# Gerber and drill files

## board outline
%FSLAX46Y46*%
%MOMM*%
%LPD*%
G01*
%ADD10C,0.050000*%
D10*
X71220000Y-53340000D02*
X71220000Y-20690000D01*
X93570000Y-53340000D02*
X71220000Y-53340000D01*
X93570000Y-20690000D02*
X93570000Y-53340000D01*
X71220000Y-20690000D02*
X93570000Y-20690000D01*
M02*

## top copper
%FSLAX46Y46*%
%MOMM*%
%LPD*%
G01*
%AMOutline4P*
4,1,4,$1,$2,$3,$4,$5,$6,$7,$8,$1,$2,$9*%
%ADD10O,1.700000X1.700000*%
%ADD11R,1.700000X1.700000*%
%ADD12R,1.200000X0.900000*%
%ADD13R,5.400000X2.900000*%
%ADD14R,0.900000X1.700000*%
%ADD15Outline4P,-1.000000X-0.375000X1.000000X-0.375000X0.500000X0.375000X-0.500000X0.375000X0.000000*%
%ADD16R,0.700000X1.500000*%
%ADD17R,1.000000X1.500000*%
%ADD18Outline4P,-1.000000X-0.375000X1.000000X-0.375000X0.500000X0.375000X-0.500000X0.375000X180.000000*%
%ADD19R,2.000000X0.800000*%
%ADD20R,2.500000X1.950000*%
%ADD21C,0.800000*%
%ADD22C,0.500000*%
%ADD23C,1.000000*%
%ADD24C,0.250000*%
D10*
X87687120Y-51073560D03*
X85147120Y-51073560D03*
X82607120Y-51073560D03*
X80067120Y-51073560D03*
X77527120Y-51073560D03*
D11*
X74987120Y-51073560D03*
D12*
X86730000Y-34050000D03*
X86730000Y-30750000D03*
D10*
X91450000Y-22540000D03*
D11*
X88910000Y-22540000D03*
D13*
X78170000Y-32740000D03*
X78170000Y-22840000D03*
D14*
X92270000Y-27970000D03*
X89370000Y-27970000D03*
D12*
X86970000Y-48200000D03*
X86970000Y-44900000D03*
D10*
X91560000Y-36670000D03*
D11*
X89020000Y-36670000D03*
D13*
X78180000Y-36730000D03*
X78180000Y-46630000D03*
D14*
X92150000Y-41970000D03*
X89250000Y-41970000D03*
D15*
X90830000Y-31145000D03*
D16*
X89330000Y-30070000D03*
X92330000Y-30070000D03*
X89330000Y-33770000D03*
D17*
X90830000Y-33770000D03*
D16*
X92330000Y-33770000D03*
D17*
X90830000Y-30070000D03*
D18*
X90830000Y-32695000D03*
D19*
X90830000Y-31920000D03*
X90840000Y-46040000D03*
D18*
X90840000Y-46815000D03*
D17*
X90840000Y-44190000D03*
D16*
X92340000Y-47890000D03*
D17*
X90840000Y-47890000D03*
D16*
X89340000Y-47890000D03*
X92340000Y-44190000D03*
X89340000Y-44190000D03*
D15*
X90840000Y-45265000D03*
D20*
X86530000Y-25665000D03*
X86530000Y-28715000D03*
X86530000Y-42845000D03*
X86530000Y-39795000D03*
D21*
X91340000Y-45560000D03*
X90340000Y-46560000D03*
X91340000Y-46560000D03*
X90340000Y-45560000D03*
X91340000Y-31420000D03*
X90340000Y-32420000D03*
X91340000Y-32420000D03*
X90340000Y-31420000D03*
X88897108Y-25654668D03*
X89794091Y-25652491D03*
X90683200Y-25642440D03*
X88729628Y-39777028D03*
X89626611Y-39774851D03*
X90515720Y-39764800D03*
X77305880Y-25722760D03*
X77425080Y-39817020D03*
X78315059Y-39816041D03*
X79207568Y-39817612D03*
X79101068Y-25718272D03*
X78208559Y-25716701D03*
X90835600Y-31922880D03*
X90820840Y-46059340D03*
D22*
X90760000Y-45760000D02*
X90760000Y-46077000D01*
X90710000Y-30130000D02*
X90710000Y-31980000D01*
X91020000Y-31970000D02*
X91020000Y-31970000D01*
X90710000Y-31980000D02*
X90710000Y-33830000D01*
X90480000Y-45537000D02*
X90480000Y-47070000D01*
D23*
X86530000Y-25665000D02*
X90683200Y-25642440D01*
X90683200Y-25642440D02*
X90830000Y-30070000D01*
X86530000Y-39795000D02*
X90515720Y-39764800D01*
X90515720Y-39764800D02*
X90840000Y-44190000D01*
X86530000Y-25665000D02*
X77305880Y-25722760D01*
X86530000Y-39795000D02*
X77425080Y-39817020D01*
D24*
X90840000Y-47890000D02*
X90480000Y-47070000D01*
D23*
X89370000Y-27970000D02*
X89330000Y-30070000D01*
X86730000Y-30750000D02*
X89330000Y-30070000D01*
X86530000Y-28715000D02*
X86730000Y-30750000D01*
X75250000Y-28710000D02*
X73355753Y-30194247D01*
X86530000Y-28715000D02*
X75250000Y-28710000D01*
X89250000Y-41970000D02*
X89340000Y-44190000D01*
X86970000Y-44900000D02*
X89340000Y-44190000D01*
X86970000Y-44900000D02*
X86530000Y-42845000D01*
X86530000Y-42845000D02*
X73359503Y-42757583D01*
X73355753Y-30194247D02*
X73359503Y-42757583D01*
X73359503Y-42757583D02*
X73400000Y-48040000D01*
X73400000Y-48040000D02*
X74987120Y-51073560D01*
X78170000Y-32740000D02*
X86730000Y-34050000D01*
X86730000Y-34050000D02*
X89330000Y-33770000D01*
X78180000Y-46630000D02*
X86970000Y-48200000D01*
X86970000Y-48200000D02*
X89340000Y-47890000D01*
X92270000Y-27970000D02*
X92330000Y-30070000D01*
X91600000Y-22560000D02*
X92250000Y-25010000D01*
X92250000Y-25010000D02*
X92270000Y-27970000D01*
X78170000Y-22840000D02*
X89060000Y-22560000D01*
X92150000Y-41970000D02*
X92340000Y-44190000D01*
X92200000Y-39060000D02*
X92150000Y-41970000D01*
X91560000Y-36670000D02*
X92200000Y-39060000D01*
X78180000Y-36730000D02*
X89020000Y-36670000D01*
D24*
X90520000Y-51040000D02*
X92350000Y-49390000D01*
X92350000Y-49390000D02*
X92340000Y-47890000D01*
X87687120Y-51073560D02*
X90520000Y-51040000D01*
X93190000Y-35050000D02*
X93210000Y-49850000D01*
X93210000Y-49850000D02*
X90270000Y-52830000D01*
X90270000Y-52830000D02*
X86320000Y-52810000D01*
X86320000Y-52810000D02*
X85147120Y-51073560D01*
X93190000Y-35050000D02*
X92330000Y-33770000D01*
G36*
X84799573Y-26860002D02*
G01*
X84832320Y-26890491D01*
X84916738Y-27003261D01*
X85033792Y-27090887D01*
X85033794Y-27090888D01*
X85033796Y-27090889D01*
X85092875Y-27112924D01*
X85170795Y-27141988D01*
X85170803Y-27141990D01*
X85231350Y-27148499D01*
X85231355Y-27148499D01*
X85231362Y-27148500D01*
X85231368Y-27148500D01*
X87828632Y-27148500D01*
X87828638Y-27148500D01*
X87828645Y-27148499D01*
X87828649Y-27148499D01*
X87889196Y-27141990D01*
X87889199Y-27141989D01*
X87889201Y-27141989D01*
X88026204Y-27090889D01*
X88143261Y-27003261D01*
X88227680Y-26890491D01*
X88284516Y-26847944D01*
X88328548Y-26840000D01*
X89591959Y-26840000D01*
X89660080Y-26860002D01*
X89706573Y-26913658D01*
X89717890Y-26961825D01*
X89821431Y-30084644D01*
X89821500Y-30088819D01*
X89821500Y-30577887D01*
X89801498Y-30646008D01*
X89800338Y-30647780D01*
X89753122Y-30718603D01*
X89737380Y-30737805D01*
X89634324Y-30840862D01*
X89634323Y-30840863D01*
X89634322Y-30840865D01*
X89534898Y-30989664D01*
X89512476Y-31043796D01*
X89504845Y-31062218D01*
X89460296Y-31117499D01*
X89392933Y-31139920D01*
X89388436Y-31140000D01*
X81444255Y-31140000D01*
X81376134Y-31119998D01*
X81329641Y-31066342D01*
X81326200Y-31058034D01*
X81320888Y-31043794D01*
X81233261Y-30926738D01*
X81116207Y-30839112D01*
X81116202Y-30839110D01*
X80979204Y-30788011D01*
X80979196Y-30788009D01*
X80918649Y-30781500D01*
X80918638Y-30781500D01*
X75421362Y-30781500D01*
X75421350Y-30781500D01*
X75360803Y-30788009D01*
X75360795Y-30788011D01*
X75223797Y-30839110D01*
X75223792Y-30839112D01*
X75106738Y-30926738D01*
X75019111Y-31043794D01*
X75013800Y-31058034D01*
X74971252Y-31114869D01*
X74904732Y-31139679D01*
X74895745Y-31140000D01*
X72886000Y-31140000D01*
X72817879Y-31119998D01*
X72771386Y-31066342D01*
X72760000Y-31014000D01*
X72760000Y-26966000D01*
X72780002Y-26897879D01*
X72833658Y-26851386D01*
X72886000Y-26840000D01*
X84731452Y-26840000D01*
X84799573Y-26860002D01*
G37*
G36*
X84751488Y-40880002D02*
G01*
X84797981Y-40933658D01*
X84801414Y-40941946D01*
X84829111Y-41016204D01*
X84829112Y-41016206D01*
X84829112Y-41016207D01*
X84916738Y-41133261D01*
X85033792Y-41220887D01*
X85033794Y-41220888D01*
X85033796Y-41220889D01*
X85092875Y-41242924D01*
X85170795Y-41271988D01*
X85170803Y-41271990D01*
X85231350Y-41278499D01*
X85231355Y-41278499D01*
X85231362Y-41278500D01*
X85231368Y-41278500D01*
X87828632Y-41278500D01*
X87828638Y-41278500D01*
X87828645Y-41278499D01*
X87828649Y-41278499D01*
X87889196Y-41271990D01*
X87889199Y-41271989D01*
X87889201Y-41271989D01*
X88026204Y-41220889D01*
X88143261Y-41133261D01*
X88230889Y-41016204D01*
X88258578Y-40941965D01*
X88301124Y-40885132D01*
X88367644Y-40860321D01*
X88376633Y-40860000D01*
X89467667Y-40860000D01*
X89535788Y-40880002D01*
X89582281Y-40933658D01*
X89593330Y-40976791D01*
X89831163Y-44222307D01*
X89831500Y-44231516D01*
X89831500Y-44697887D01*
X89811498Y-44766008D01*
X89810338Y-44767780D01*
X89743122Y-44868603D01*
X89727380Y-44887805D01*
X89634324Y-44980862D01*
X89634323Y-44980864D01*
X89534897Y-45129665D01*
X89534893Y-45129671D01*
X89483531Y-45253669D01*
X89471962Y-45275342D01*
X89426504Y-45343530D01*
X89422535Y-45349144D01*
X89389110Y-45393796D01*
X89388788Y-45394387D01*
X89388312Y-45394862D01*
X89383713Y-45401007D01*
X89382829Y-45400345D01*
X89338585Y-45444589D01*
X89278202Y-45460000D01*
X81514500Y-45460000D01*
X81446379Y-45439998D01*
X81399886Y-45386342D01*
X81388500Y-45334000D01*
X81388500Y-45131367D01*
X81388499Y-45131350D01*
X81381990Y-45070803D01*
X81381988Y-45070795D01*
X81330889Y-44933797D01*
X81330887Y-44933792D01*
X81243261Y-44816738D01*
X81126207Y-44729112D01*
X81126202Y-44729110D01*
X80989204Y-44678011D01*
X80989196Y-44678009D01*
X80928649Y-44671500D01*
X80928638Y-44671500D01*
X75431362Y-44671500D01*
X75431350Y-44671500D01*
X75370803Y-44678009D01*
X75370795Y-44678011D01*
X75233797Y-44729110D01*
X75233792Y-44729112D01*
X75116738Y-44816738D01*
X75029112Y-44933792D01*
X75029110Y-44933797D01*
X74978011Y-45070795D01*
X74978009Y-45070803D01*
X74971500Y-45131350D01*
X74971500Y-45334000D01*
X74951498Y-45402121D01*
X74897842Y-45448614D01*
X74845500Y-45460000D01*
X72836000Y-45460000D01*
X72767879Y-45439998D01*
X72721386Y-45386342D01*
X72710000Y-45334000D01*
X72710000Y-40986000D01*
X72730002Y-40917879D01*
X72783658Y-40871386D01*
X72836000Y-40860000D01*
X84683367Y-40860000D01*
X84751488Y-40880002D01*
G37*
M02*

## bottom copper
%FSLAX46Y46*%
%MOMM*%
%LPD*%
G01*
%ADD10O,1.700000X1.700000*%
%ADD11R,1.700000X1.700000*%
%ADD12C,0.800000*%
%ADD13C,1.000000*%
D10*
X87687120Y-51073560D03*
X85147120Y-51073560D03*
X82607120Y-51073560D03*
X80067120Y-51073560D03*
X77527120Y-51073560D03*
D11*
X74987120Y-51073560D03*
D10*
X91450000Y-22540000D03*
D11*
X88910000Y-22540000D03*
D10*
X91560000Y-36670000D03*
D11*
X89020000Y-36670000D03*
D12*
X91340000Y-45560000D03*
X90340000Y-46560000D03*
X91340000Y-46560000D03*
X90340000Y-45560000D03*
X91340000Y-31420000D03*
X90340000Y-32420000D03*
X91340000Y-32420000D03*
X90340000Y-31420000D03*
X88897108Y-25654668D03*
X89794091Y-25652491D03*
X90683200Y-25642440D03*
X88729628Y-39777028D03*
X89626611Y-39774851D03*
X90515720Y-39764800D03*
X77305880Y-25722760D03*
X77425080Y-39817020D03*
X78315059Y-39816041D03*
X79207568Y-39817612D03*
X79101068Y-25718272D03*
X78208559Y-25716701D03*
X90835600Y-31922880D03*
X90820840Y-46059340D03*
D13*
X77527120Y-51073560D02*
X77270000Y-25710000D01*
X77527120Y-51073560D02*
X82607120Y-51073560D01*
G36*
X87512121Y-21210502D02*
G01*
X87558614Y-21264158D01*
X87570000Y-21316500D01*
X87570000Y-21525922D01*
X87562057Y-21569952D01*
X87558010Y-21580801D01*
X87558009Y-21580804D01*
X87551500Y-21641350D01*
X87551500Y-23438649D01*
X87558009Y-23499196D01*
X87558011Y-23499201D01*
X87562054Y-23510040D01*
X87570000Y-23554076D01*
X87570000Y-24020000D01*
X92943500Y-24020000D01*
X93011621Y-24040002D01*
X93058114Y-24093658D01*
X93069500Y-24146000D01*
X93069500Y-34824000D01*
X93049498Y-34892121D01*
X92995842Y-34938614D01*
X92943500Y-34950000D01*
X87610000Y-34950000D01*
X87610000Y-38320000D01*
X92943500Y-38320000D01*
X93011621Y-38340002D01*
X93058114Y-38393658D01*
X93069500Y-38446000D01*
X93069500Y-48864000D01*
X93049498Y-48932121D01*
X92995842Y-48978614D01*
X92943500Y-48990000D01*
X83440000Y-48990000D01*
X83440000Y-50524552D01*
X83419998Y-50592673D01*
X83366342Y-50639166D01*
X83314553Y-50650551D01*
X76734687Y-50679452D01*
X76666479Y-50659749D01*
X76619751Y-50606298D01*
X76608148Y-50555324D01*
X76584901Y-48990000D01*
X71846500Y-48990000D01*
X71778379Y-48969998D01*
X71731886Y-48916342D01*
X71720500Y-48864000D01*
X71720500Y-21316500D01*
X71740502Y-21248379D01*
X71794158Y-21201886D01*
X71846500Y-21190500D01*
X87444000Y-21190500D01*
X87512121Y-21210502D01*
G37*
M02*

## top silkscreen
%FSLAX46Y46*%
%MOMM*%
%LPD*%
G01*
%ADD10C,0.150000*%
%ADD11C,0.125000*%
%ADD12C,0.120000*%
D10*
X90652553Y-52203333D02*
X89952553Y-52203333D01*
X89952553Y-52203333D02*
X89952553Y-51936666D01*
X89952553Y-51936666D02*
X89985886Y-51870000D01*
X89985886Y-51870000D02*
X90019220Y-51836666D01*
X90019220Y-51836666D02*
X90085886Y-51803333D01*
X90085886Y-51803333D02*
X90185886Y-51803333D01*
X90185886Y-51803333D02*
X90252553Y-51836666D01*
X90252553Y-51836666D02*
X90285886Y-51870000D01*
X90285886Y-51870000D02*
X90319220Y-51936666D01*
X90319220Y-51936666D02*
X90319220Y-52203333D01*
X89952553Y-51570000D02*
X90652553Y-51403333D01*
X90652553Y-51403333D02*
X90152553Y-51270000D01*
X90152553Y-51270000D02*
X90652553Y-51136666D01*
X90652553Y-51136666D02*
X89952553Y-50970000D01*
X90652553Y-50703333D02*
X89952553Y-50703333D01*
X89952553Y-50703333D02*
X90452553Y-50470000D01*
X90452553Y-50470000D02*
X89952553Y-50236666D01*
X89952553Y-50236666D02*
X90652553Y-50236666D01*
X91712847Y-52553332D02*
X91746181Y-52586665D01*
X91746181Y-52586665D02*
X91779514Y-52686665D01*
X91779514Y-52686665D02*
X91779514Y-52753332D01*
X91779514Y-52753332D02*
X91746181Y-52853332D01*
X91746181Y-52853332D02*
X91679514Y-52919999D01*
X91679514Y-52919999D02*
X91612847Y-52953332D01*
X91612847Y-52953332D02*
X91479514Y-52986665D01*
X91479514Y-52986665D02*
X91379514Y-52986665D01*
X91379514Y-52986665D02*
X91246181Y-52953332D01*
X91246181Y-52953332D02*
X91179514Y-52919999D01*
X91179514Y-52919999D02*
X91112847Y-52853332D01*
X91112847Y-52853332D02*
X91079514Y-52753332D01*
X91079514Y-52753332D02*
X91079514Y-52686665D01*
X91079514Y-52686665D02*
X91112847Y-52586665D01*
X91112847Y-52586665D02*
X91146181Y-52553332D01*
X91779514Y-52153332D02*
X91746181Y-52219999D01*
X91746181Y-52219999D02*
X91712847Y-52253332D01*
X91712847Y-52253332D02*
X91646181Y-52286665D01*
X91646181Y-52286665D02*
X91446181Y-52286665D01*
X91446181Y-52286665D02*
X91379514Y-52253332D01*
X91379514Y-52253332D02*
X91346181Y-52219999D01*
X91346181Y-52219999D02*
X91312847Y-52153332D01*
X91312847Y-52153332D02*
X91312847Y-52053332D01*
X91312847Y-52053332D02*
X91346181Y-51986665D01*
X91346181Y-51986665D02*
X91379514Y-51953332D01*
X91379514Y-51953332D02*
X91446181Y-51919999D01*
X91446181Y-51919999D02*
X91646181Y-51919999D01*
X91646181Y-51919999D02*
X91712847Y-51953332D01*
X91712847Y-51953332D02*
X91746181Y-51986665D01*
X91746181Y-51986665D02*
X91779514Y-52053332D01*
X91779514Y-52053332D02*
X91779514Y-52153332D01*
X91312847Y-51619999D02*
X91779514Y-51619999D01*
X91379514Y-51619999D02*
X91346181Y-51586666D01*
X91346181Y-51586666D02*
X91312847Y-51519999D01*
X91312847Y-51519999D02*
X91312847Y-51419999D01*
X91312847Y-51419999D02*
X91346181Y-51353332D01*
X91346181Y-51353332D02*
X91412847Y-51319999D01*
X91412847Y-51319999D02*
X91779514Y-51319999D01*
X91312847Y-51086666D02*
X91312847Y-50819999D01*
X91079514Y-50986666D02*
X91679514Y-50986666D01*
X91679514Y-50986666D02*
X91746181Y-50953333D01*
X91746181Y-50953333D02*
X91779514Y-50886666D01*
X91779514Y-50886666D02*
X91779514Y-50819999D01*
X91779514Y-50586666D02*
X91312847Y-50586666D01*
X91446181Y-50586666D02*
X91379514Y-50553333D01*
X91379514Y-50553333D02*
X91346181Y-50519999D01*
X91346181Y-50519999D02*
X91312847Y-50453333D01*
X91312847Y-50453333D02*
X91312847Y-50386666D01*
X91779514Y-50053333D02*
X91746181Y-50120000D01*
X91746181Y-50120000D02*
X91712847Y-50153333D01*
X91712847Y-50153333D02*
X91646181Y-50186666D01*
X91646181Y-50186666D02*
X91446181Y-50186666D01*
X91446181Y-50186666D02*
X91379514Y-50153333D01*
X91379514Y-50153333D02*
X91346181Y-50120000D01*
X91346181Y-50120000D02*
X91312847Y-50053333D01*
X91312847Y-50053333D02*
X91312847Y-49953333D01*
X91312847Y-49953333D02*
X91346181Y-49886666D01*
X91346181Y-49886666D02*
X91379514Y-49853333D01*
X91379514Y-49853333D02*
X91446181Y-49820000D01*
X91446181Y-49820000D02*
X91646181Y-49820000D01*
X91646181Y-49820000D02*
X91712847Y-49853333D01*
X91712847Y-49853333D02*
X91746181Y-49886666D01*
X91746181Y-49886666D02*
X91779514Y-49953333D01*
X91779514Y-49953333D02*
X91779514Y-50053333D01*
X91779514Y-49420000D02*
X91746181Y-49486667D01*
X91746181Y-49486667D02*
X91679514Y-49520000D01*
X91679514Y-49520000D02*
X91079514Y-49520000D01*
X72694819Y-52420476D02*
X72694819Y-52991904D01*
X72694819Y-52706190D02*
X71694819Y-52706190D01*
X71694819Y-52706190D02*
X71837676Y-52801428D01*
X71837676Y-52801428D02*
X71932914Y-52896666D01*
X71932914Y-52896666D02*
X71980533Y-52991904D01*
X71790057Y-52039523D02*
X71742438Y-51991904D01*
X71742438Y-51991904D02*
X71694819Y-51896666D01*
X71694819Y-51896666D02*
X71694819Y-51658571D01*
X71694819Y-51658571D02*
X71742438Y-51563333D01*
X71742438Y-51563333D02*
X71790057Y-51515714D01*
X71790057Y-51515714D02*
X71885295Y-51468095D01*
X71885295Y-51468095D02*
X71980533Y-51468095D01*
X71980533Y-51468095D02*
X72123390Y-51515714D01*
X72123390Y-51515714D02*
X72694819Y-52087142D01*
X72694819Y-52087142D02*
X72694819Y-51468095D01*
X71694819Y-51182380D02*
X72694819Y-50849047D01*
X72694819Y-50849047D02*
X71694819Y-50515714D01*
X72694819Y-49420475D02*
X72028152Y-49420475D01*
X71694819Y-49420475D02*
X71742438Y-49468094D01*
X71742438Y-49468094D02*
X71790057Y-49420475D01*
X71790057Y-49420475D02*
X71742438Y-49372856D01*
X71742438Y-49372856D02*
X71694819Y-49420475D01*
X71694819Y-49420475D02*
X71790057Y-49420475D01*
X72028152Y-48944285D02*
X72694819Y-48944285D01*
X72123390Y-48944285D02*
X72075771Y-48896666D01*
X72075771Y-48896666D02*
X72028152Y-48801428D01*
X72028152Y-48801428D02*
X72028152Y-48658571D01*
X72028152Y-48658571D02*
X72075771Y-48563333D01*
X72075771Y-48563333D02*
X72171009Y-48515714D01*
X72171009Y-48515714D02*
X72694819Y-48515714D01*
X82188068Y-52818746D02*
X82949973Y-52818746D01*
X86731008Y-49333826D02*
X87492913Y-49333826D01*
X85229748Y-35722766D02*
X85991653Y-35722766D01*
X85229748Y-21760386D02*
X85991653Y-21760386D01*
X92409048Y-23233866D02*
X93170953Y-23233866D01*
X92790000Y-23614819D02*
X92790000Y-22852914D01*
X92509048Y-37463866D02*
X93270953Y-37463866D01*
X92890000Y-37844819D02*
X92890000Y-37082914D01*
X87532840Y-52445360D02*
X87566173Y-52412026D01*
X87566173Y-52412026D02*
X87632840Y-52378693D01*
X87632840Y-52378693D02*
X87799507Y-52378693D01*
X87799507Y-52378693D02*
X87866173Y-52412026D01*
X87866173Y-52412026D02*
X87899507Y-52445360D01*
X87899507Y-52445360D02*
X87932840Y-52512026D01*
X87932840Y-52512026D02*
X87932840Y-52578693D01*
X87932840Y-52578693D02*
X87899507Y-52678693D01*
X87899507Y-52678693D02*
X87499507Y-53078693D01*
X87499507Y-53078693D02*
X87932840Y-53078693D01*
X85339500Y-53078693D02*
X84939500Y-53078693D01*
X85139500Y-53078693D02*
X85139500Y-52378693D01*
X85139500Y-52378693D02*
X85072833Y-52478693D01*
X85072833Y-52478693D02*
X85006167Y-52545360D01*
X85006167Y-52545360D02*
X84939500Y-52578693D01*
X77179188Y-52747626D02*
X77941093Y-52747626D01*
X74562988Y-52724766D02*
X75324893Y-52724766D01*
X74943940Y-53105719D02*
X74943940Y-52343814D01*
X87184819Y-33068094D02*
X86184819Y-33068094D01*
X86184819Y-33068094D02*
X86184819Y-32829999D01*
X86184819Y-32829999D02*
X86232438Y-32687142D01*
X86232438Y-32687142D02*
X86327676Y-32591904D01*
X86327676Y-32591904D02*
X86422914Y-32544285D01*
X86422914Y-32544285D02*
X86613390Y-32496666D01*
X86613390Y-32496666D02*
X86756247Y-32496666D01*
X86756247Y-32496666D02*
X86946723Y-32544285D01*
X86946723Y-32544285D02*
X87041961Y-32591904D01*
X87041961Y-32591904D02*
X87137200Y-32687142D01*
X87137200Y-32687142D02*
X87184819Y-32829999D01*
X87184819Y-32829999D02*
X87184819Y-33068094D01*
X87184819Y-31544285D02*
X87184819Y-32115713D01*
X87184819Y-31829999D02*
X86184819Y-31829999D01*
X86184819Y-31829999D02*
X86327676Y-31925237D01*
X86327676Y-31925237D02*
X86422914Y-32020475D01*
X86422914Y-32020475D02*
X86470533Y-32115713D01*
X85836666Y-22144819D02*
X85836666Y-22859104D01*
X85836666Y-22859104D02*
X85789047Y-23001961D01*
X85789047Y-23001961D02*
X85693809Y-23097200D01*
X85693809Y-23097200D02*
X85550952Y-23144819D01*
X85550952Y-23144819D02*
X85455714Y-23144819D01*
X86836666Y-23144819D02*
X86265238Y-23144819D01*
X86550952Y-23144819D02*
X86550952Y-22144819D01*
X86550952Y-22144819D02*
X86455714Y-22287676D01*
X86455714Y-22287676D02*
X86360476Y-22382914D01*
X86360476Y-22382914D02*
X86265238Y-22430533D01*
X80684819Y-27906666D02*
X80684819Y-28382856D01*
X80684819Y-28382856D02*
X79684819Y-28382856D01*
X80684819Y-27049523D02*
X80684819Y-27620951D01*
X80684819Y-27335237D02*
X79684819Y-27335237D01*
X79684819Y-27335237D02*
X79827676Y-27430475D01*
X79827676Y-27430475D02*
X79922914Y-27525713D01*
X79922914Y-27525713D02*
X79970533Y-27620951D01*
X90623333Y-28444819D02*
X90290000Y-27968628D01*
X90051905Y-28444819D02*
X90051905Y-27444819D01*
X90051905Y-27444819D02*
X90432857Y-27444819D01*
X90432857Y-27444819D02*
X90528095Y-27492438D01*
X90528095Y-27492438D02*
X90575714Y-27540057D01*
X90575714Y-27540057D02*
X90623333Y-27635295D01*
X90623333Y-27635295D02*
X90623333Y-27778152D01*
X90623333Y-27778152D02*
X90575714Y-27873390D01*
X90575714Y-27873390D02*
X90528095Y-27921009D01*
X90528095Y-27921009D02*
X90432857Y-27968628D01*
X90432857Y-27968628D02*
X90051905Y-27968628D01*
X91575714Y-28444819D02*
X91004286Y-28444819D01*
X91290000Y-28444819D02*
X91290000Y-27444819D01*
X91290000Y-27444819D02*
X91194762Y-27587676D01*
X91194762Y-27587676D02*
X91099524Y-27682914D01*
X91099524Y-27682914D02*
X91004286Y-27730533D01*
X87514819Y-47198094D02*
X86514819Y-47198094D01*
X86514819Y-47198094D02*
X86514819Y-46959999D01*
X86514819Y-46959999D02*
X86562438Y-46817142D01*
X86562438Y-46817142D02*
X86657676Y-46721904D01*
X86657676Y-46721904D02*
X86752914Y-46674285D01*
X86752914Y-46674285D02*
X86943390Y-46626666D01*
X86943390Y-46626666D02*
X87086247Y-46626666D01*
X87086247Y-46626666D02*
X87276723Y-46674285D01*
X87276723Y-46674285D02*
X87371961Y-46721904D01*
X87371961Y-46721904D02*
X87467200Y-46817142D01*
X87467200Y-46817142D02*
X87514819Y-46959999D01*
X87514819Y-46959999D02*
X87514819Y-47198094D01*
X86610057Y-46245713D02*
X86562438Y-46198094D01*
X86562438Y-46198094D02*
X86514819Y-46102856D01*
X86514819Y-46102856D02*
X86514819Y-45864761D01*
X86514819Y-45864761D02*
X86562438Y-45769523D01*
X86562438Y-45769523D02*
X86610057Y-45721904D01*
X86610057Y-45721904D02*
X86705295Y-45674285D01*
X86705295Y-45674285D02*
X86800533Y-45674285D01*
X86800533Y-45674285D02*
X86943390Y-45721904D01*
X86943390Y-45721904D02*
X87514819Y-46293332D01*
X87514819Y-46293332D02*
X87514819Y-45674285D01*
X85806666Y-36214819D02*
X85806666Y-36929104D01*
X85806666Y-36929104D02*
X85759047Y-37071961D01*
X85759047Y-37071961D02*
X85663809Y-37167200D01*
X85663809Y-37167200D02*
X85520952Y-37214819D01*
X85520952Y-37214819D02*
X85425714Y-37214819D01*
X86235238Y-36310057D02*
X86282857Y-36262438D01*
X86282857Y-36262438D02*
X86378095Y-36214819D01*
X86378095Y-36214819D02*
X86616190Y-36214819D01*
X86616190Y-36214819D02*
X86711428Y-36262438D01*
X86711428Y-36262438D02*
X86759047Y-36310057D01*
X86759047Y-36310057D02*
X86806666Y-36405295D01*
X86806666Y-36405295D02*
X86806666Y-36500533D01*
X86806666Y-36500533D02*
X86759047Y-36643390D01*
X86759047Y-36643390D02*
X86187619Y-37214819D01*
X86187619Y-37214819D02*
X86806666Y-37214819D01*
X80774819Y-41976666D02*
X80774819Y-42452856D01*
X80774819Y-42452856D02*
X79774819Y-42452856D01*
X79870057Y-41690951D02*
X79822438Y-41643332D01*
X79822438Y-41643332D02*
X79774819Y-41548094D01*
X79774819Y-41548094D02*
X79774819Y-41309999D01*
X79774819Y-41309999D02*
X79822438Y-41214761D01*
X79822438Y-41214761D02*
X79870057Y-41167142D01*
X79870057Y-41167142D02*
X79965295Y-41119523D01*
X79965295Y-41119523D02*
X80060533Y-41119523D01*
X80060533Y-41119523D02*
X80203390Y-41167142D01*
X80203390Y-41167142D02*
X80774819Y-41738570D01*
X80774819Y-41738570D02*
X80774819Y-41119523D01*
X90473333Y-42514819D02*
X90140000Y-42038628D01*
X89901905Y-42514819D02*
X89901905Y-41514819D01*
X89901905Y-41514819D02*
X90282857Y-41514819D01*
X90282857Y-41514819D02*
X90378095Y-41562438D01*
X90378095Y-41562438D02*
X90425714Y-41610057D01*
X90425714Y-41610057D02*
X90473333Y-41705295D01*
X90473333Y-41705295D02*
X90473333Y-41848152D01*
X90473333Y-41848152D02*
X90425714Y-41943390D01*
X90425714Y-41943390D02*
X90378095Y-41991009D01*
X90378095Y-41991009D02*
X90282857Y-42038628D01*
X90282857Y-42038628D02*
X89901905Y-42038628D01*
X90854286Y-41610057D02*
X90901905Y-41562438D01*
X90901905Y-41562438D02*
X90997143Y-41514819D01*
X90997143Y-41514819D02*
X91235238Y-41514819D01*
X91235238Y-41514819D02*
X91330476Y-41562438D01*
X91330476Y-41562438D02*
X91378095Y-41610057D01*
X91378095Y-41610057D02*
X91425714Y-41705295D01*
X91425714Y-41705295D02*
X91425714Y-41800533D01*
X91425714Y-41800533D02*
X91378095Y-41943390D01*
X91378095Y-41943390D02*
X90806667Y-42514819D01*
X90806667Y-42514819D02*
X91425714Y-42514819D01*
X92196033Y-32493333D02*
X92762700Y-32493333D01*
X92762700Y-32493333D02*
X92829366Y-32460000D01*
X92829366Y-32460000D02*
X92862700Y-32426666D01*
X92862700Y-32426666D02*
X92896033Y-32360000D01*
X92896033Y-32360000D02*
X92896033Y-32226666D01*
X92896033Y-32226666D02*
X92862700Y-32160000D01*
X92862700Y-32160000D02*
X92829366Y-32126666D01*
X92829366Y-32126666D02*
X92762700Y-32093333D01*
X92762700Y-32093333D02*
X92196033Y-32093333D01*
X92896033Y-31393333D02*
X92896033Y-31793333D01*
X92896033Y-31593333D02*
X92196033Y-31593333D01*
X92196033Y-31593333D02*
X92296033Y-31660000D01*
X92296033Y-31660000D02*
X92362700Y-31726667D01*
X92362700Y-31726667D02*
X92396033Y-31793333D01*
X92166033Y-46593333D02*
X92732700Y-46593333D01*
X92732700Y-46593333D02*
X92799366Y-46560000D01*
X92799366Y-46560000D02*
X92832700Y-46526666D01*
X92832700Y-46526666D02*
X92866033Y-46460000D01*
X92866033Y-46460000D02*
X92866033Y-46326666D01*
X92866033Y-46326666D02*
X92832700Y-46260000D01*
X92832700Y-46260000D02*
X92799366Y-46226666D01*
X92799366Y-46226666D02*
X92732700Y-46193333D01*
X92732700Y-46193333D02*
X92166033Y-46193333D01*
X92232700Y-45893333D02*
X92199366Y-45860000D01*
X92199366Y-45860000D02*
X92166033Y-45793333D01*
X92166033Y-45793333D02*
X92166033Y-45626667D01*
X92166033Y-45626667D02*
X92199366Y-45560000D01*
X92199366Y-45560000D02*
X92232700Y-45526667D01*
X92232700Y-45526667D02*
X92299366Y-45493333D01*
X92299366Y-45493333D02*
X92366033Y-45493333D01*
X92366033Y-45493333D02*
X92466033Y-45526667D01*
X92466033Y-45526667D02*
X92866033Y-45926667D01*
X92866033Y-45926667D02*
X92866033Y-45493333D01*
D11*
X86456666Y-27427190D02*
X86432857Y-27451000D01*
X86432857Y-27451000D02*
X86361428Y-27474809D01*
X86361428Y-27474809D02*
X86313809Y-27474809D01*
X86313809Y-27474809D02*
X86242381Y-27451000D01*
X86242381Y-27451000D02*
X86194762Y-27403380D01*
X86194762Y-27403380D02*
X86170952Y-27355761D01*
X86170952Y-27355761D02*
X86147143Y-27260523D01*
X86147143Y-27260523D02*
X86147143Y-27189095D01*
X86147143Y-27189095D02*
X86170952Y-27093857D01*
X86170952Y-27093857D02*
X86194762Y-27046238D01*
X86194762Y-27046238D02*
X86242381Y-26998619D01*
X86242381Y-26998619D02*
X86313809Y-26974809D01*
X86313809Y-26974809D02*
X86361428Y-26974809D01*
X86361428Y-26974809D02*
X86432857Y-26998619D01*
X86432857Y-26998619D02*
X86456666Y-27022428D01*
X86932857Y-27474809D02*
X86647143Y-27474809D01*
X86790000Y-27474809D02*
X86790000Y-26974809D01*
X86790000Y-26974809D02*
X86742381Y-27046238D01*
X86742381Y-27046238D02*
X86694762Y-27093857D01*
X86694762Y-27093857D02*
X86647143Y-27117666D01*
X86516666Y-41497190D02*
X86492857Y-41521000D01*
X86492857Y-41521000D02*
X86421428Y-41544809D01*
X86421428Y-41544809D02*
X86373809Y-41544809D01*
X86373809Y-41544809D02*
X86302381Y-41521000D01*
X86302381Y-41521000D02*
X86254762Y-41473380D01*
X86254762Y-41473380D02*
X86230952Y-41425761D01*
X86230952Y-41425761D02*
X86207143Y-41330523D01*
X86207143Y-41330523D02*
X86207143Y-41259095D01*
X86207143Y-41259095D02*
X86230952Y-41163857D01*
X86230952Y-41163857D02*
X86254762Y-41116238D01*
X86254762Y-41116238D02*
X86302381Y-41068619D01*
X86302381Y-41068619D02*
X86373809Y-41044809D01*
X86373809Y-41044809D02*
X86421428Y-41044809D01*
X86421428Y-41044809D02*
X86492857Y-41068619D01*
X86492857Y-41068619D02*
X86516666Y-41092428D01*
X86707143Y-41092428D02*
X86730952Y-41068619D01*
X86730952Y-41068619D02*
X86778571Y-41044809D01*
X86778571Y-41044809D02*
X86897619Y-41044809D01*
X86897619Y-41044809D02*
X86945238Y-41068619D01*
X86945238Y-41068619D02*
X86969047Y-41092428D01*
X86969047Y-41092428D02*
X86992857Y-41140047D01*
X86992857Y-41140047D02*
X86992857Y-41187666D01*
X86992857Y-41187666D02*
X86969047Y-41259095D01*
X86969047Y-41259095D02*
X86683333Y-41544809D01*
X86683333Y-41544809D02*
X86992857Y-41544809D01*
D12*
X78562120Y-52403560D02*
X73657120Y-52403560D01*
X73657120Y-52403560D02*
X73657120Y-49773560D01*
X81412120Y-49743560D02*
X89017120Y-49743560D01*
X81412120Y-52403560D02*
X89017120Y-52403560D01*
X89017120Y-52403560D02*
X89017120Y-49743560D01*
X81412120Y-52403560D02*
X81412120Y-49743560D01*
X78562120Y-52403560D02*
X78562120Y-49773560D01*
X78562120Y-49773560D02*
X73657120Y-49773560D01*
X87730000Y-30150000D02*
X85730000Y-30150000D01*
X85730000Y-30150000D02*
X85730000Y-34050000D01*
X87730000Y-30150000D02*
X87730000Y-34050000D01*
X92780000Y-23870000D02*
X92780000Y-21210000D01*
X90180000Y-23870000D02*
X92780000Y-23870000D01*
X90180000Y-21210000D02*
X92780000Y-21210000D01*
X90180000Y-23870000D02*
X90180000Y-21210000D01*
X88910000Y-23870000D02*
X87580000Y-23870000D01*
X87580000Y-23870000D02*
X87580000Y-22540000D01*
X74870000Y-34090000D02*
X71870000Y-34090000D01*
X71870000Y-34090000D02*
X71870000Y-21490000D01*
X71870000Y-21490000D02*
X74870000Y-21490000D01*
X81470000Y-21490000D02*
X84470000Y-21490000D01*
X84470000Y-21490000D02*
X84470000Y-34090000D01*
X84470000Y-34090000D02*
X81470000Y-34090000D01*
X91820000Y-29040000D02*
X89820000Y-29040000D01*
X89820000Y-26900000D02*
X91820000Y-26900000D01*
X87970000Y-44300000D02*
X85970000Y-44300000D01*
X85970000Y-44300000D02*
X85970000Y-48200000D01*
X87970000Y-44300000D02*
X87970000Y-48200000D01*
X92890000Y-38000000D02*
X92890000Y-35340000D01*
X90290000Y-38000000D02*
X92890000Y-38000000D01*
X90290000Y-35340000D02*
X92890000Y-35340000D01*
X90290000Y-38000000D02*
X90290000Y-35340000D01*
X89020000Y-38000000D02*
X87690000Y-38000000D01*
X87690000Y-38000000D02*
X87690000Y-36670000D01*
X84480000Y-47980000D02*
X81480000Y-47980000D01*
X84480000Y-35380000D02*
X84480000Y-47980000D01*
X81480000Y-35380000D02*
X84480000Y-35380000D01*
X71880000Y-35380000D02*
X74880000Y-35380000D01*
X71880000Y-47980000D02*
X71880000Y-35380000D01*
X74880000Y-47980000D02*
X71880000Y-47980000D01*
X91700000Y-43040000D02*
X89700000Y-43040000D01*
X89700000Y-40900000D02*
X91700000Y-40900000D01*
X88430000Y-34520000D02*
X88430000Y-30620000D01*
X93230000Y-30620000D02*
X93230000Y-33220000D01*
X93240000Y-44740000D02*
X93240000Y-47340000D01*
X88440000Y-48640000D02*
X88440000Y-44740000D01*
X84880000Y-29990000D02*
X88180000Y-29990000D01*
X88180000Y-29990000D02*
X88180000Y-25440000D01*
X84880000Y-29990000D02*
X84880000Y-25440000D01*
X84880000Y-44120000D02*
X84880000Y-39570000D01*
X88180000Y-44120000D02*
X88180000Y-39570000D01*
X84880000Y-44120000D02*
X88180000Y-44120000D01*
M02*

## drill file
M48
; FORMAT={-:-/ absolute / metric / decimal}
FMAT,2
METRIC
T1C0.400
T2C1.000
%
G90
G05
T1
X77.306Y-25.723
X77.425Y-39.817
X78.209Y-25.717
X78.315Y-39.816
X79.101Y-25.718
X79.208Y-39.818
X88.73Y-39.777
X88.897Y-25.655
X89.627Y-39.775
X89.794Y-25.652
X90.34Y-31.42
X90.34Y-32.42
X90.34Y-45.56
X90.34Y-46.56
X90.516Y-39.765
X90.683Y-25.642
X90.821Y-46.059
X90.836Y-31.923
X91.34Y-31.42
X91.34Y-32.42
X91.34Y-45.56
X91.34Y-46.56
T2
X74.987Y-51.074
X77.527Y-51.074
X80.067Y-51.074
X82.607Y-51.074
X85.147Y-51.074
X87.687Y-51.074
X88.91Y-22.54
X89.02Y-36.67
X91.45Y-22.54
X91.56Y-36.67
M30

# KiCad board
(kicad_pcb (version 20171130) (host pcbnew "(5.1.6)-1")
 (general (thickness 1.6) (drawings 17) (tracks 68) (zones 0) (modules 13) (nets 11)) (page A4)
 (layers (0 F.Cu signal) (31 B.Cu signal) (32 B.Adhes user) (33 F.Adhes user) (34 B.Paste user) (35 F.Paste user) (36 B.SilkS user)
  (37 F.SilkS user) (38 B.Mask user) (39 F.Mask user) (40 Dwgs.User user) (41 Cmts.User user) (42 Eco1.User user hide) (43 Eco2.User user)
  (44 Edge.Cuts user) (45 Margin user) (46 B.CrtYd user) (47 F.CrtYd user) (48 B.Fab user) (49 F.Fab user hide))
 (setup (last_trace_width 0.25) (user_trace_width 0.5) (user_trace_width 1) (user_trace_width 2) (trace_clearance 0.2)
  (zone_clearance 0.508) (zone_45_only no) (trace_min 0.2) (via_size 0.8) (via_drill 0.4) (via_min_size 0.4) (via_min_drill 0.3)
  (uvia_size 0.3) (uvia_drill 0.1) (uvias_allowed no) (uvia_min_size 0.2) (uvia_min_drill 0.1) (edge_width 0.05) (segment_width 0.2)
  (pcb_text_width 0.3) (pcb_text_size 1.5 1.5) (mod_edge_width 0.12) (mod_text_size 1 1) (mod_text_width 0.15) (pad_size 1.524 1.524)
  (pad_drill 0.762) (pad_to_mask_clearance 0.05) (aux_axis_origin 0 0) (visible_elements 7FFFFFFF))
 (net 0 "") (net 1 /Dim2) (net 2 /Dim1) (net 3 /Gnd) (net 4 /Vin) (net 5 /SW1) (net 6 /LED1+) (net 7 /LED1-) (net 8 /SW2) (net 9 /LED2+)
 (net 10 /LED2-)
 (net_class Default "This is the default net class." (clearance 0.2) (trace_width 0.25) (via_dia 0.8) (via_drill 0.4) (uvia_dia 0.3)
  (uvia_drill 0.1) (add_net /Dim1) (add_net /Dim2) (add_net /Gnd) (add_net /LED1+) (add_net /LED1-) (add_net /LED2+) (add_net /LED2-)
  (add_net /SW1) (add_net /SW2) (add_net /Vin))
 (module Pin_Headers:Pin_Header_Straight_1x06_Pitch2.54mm (layer F.Cu) (at 74.98712 51.07356 90)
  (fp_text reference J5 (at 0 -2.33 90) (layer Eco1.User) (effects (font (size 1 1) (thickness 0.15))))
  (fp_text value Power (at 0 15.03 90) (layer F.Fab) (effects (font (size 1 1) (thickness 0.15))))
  (fp_line (start -1.33 3.575) (end -1.33 -1.33) (layer F.SilkS) (width 0.12))
  (fp_line (start -1.33 -1.33) (end 1.3 -1.33) (layer F.SilkS) (width 0.12))
  (fp_line (start 1.33 6.425) (end 1.33 14.03) (layer F.SilkS) (width 0.12))
  (fp_line (start -1.33 6.425) (end -1.33 14.03) (layer F.SilkS) (width 0.12))
  (fp_line (start -1.33 14.03) (end 1.33 14.03) (layer F.SilkS) (width 0.12))
  (fp_line (start -1.33 6.425) (end 1.33 6.425) (layer F.SilkS) (width 0.12))
  (fp_line (start -1.33 3.575) (end 1.3 3.575) (layer F.SilkS) (width 0.12))
  (fp_line (start 1.3 3.575) (end 1.3 -1.33) (layer F.SilkS) (width 0.12))
  (pad 6 thru_hole oval (at 0 12.7 90) (size 1.7 1.7) (drill 1) (layers *.Cu *.Mask) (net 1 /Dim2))
  (pad 5 thru_hole oval (at 0 10.16 90) (size 1.7 1.7) (drill 1) (layers *.Cu *.Mask) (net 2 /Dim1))
  (pad 4 thru_hole oval (at 0 7.62 90) (size 1.7 1.7) (drill 1) (layers *.Cu *.Mask) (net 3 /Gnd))
  (pad 3 thru_hole oval (at 0 5.08 90) (size 1.7 1.7) (drill 1) (layers *.Cu *.Mask) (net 3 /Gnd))
  (pad 2 thru_hole oval (at 0 2.54 90) (size 1.7 1.7) (drill 1) (layers *.Cu *.Mask) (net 3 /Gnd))
  (pad 1 thru_hole rect (at 0 0 90) (size 1.7 1.7) (drill 1) (layers *.Cu *.Mask) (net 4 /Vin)))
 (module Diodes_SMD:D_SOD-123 (layer F.Cu) (at 86.73 32.4 270)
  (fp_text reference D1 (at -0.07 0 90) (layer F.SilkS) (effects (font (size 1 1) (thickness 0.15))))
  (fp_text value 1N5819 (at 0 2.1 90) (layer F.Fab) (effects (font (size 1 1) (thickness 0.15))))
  (fp_line (start -2.25 -1) (end -2.25 1) (layer F.SilkS) (width 0.12))
  (fp_line (start -2.25 1) (end 1.65 1) (layer F.SilkS) (width 0.12))
  (fp_line (start -2.25 -1) (end 1.65 -1) (layer F.SilkS) (width 0.12))
  (pad 2 smd rect (at 1.65 0 270) (size 0.9 1.2) (layers F.Cu F.Paste F.Mask) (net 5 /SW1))
  (pad 1 smd rect (at -1.65 0 270) (size 0.9 1.2) (layers F.Cu F.Paste F.Mask) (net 4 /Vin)))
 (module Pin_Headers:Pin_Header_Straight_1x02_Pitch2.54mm (layer F.Cu) (at 88.91 22.54 90)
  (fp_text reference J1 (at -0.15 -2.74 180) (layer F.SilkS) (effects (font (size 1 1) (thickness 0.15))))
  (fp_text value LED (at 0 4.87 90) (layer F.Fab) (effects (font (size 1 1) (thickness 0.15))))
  (fp_line (start -1.33 3.87) (end 1.33 3.87) (layer F.SilkS) (width 0.12))
  (fp_line (start -1.33 1.27) (end -1.33 3.87) (layer F.SilkS) (width 0.12))
  (fp_line (start 1.33 1.27) (end 1.33 3.87) (layer F.SilkS) (width 0.12))
  (fp_line (start -1.33 1.27) (end 1.33 1.27) (layer F.SilkS) (width 0.12))
  (fp_line (start -1.33 0) (end -1.33 -1.33) (layer F.SilkS) (width 0.12))
  (fp_line (start -1.33 -1.33) (end 0 -1.33) (layer F.SilkS) (width 0.12))
  (pad 2 thru_hole oval (at 0 2.54 90) (size 1.7 1.7) (drill 1) (layers *.Cu *.Mask) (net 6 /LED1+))
  (pad 1 thru_hole rect (at 0 0 90) (size 1.7 1.7) (drill 1) (layers *.Cu *.Mask) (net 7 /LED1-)))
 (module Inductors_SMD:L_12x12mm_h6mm (layer F.Cu) (at 78.17 27.79 270)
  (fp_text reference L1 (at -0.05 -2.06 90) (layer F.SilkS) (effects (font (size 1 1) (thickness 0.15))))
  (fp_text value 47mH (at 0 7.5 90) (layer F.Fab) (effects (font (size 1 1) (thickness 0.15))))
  (fp_line (start 6.3 3.3) (end 6.3 6.3) (layer F.SilkS) (width 0.12))
  (fp_line (start 6.3 6.3) (end -6.3 6.3) (layer F.SilkS) (width 0.12))
  (fp_line (start -6.3 6.3) (end -6.3 3.3) (layer F.SilkS) (width 0.12))
  (fp_line (start -6.3 -3.3) (end -6.3 -6.3) (layer F.SilkS) (width 0.12))
  (fp_line (start -6.3 -6.3) (end 6.3 -6.3) (layer F.SilkS) (width 0.12))
  (fp_line (start 6.3 -6.3) (end 6.3 -3.3) (layer F.SilkS) (width 0.12))
  (pad 2 smd rect (at 4.95 0 270) (size 2.9 5.4) (layers F.Cu F.Paste F.Mask) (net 5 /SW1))
  (pad 1 smd rect (at -4.95 0 270) (size 2.9 5.4) (layers F.Cu F.Paste F.Mask) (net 7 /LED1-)))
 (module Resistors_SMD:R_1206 (layer F.Cu) (at 90.82 27.97)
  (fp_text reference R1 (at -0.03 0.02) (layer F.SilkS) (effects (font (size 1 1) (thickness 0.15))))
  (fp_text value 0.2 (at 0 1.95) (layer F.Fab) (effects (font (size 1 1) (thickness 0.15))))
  (fp_line (start 1 1.07) (end -1 1.07) (layer F.SilkS) (width 0.12))
  (fp_line (start -1 -1.07) (end 1 -1.07) (layer F.SilkS) (width 0.12))
  (pad 2 smd rect (at 1.45 0) (size 0.9 1.7) (layers F.Cu F.Paste F.Mask) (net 6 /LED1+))
  (pad 1 smd rect (at -1.45 0) (size 0.9 1.7) (layers F.Cu F.Paste F.Mask) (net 4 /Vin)))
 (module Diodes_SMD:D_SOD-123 (layer F.Cu) (at 86.97 46.55 270)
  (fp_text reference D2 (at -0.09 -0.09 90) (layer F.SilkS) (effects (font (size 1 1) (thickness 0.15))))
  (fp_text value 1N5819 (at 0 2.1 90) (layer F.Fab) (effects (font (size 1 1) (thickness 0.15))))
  (fp_line (start -2.25 -1) (end -2.25 1) (layer F.SilkS) (width 0.12))
  (fp_line (start -2.25 1) (end 1.65 1) (layer F.SilkS) (width 0.12))
  (fp_line (start -2.25 -1) (end 1.65 -1) (layer F.SilkS) (width 0.12))
  (pad 2 smd rect (at 1.65 0 270) (size 0.9 1.2) (layers F.Cu F.Paste F.Mask) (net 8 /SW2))
  (pad 1 smd rect (at -1.65 0 270) (size 0.9 1.2) (layers F.Cu F.Paste F.Mask) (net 4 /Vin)))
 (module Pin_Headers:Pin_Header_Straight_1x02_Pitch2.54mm (layer F.Cu) (at 89.02 36.67 90)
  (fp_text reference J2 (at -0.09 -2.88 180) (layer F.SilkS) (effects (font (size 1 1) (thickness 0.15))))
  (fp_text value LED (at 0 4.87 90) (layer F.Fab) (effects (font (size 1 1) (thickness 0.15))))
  (fp_line (start -1.33 3.87) (end 1.33 3.87) (layer F.SilkS) (width 0.12))
  (fp_line (start -1.33 1.27) (end -1.33 3.87) (layer F.SilkS) (width 0.12))
  (fp_line (start 1.33 1.27) (end 1.33 3.87) (layer F.SilkS) (width 0.12))
  (fp_line (start -1.33 1.27) (end 1.33 1.27) (layer F.SilkS) (width 0.12))
  (fp_line (start -1.33 0) (end -1.33 -1.33) (layer F.SilkS) (width 0.12))
  (fp_line (start -1.33 -1.33) (end 0 -1.33) (layer F.SilkS) (width 0.12))
  (pad 2 thru_hole oval (at 0 2.54 90) (size 1.7 1.7) (drill 1) (layers *.Cu *.Mask) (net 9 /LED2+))
  (pad 1 thru_hole rect (at 0 0 90) (size 1.7 1.7) (drill 1) (layers *.Cu *.Mask) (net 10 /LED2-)))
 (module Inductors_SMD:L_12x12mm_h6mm (layer F.Cu) (at 78.18 41.68 270)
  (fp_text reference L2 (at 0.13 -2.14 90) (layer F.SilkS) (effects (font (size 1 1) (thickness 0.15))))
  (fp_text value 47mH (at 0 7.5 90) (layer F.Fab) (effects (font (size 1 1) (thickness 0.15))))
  (fp_line (start 6.3 -6.3) (end 6.3 -3.3) (layer F.SilkS) (width 0.12))
  (fp_line (start -6.3 -6.3) (end 6.3 -6.3) (layer F.SilkS) (width 0.12))
  (fp_line (start -6.3 -3.3) (end -6.3 -6.3) (layer F.SilkS) (width 0.12))
  (fp_line (start -6.3 6.3) (end -6.3 3.3) (layer F.SilkS) (width 0.12))
  (fp_line (start 6.3 6.3) (end -6.3 6.3) (layer F.SilkS) (width 0.12))
  (fp_line (start 6.3 3.3) (end 6.3 6.3) (layer F.SilkS) (width 0.12))
  (pad 1 smd rect (at -4.95 0 270) (size 2.9 5.4) (layers F.Cu F.Paste F.Mask) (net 10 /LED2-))
  (pad 2 smd rect (at 4.95 0 270) (size 2.9 5.4) (layers F.Cu F.Paste F.Mask) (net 8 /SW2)))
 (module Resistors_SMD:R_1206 (layer F.Cu) (at 90.7 41.97)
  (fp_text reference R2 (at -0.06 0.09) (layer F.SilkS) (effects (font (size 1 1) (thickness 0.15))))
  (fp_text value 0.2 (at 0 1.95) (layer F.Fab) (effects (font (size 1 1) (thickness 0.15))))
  (fp_line (start 1 1.07) (end -1 1.07) (layer F.SilkS) (width 0.12))
  (fp_line (start -1 -1.07) (end 1 -1.07) (layer F.SilkS) (width 0.12))
  (pad 2 smd rect (at 1.45 0) (size 0.9 1.7) (layers F.Cu F.Paste F.Mask) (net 9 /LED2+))
  (pad 1 smd rect (at -1.45 0) (size 0.9 1.7) (layers F.Cu F.Paste F.Mask) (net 4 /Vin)))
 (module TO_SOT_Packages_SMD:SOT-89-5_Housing (layer F.Cu) (at 90.83 31.92 90)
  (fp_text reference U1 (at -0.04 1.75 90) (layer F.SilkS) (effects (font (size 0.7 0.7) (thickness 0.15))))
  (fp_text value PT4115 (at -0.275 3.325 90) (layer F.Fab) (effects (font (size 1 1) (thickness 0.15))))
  (fp_line (start -2.6 -2.4) (end 1.3 -2.4) (layer F.SilkS) (width 0.12))
  (fp_line (start 1.3 2.4) (end -1.3 2.4) (layer F.SilkS) (width 0.12))
  (pad 2 smd trapezoid (at 0.775 0) (size 1.5 0.75) (rect_delta 0 0.5) (layers F.Cu F.Paste F.Mask) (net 3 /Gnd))
  (pad 5 smd rect (at 1.85 -1.5) (size 0.7 1.5) (layers F.Cu F.Paste F.Mask) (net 4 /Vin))
  (pad 4 smd rect (at 1.85 1.5) (size 0.7 1.5) (layers F.Cu F.Paste F.Mask) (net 6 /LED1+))
  (pad 1 smd rect (at -1.85 -1.5) (size 0.7 1.5) (layers F.Cu F.Paste F.Mask) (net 5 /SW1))
  (pad 2 smd rect (at -1.85 0) (size 1 1.5) (layers F.Cu F.Paste F.Mask) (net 3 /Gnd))
  (pad 3 smd rect (at -1.85 1.5) (size 0.7 1.5) (layers F.Cu F.Paste F.Mask) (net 2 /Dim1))
  (pad 2 smd rect (at 1.85 0) (size 1 1.5) (layers F.Cu F.Paste F.Mask) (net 3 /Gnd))
  (pad 2 smd trapezoid (at -0.775 0 180) (size 1.5 0.75) (rect_delta 0 0.5) (layers F.Cu F.Paste F.Mask) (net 3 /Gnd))
  (pad 2 smd rect (at 0 0) (size 2 0.8) (layers F.Cu F.Paste F.Mask) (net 3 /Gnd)))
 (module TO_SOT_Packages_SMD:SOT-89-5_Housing (layer F.Cu) (at 90.84 46.04 90)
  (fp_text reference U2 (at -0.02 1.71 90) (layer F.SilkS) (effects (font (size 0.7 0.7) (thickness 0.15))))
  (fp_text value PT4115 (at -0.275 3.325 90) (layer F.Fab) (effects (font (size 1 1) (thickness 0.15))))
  (fp_line (start 1.3 2.4) (end -1.3 2.4) (layer F.SilkS) (width 0.12))
  (fp_line (start -2.6 -2.4) (end 1.3 -2.4) (layer F.SilkS) (width 0.12))
  (pad 2 smd rect (at 0 0) (size 2 0.8) (layers F.Cu F.Paste F.Mask) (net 3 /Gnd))
  (pad 2 smd trapezoid (at -0.775 0 180) (size 1.5 0.75) (rect_delta 0 0.5) (layers F.Cu F.Paste F.Mask) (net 3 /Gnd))
  (pad 2 smd rect (at 1.85 0) (size 1 1.5) (layers F.Cu F.Paste F.Mask) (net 3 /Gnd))
  (pad 3 smd rect (at -1.85 1.5) (size 0.7 1.5) (layers F.Cu F.Paste F.Mask) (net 1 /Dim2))
  (pad 2 smd rect (at -1.85 0) (size 1 1.5) (layers F.Cu F.Paste F.Mask) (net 3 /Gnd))
  (pad 1 smd rect (at -1.85 -1.5) (size 0.7 1.5) (layers F.Cu F.Paste F.Mask) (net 8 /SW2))
  (pad 4 smd rect (at 1.85 1.5) (size 0.7 1.5) (layers F.Cu F.Paste F.Mask) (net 9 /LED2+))
  (pad 5 smd rect (at 1.85 -1.5) (size 0.7 1.5) (layers F.Cu F.Paste F.Mask) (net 4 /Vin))
  (pad 2 smd trapezoid (at 0.775 0) (size 1.5 0.75) (rect_delta 0 0.5) (layers F.Cu F.Paste F.Mask) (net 3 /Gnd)))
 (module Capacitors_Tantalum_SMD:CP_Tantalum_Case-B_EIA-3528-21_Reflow (layer F.Cu) (at 86.53 27.19 90)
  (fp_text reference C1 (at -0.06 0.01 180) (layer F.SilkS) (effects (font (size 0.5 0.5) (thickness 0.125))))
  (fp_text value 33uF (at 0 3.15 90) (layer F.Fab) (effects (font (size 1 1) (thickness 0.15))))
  (fp_line (start -2.8 -1.65) (end -2.8 1.65) (layer F.SilkS) (width 0.12))
  (fp_line (start -2.8 1.65) (end 1.75 1.65) (layer F.SilkS) (width 0.12))
  (fp_line (start -2.8 -1.65) (end 1.75 -1.65) (layer F.SilkS) (width 0.12))
  (pad 2 smd rect (at 1.525 0 90) (size 1.95 2.5) (layers F.Cu F.Paste F.Mask) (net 3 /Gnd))
  (pad 1 smd rect (at -1.525 0 90) (size 1.95 2.5) (layers F.Cu F.Paste F.Mask) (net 4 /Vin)))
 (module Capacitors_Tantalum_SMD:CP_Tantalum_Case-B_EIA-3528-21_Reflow (layer F.Cu) (at 86.53 41.32 90)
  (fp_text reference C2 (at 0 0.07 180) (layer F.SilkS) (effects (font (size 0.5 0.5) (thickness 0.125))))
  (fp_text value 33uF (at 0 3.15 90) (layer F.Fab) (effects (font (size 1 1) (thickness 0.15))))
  (fp_line (start -2.8 -1.65) (end 1.75 -1.65) (layer F.SilkS) (width 0.12))
  (fp_line (start -2.8 1.65) (end 1.75 1.65) (layer F.SilkS) (width 0.12))
  (fp_line (start -2.8 -1.65) (end -2.8 1.65) (layer F.SilkS) (width 0.12))
  (pad 1 smd rect (at -1.525 0 90) (size 1.95 2.5) (layers F.Cu F.Paste F.Mask) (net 4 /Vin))
  (pad 2 smd rect (at 1.525 0 90) (size 1.95 2.5) (layers F.Cu F.Paste F.Mask) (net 3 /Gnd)))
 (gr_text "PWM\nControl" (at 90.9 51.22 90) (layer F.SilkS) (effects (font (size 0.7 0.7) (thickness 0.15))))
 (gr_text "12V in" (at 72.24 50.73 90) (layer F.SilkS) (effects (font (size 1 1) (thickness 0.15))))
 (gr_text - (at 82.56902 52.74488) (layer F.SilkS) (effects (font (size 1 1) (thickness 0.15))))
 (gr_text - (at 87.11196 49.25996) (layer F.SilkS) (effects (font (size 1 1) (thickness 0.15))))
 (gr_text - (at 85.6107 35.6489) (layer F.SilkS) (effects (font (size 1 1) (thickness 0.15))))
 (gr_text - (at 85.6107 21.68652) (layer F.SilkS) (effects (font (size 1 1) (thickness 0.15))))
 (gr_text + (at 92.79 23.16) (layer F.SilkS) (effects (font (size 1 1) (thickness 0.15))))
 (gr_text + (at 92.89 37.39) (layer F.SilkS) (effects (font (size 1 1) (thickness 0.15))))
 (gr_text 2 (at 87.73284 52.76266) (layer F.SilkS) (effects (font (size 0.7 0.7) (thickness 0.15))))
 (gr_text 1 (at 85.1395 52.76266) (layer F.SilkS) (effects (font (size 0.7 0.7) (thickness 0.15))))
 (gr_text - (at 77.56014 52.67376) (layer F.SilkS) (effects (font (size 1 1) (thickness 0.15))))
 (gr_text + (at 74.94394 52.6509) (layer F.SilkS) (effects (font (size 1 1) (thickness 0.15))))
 (gr_line (start 71.22 53.34) (end 71.22 20.69) (layer Edge.Cuts) (width 0.05))
 (gr_line (start 93.57 53.34) (end 71.22 53.34) (layer Edge.Cuts) (width 0.05))
 (gr_line (start 93.57 20.69) (end 93.57 53.34) (layer Edge.Cuts) (width 0.05))
 (gr_line (start 71.22 20.69) (end 93.57 20.69) (layer Edge.Cuts) (width 0.05))
 (segment (start 90.76 45.76) (end 90.76 46.077) (width 0.5) (layer F.Cu) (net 3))
 (segment (start 90.71 30.13) (end 90.71 31.98) (width 0.5) (layer F.Cu) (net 3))
 (segment (start 91.02 31.97) (end 91.02 31.97) (width 0.5) (layer F.Cu) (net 3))
 (via (at 91.34 45.56) (size 0.8) (drill 0.4) (layers F.Cu B.Cu) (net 3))
 (via (at 90.34 46.56) (size 0.8) (drill 0.4) (layers F.Cu B.Cu) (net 3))
 (via (at 91.34 46.56) (size 0.8) (drill 0.4) (layers F.Cu B.Cu) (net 3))
 (via (at 90.34 45.56) (size 0.8) (drill 0.4) (layers F.Cu B.Cu) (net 3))
 (via (at 91.34 31.42) (size 0.8) (drill 0.4) (layers F.Cu B.Cu) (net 3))
 (via (at 90.34 32.42) (size 0.8) (drill 0.4) (layers F.Cu B.Cu) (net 3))
 (via (at 91.34 32.42) (size 0.8) (drill 0.4) (layers F.Cu B.Cu) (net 3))
 (via (at 90.34 31.42) (size 0.8) (drill 0.4) (layers F.Cu B.Cu) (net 3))
 (via (at 88.897108 25.654668) (size 0.8) (drill 0.4) (layers F.Cu B.Cu) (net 3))
 (via (at 89.794091 25.652491) (size 0.8) (drill 0.4) (layers F.Cu B.Cu) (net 3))
 (via (at 90.6832 25.64244) (size 0.8) (drill 0.4) (layers F.Cu B.Cu) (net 3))
 (via (at 88.729628 39.777028) (size 0.8) (drill 0.4) (layers F.Cu B.Cu) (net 3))
 (via (at 89.626611 39.774851) (size 0.8) (drill 0.4) (layers F.Cu B.Cu) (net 3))
 (via (at 90.51572 39.7648) (size 0.8) (drill 0.4) (layers F.Cu B.Cu) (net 3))
 (via (at 77.30588 25.72276) (size 0.8) (drill 0.4) (layers F.Cu B.Cu) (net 3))
 (via (at 77.42508 39.81702) (size 0.8) (drill 0.4) (layers F.Cu B.Cu) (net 3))
 (via (at 78.315059 39.816041) (size 0.8) (drill 0.4) (layers F.Cu B.Cu) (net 3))
 (via (at 79.207568 39.817612) (size 0.8) (drill 0.4) (layers F.Cu B.Cu) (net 3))
 (via (at 79.101068 25.718272) (size 0.8) (drill 0.4) (layers F.Cu B.Cu) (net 3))
 (via (at 78.208559 25.716701) (size 0.8) (drill 0.4) (layers F.Cu B.Cu) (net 3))
 (segment (start 90.71 31.98) (end 90.71 33.83) (width 0.5) (layer F.Cu) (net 3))
 (via (at 90.8356 31.92288) (size 0.8) (drill 0.4) (layers F.Cu B.Cu) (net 3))
 (segment (start 90.48 45.537) (end 90.48 47.07) (width 0.5) (layer F.Cu) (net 3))
 (via (at 90.82084 46.05934) (size 0.8) (drill 0.4) (layers F.Cu B.Cu) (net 3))
 (segment (start 86.53 25.665) (end 90.6832 25.64244) (width 1) (layer F.Cu) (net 3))
 (segment (start 90.6832 25.64244) (end 90.83 30.07) (width 1) (layer F.Cu) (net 3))
 (segment (start 86.53 39.795) (end 90.51572 39.7648) (width 1) (layer F.Cu) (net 3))
 (segment (start 90.51572 39.7648) (end 90.84 44.19) (width 1) (layer F.Cu) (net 3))
 (segment (start 77.52712 51.07356) (end 77.27 25.71) (width 1) (layer B.Cu) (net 3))
 (segment (start 86.53 25.665) (end 77.30588 25.72276) (width 1) (layer F.Cu) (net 3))
 (segment (start 86.53 39.795) (end 77.42508 39.81702) (width 1) (layer F.Cu) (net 3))
 (segment (start 77.52712 51.07356) (end 82.60712 51.07356) (width 1) (layer B.Cu) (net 3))
 (segment (start 90.84 47.89) (end 90.48 47.07) (width 0.25) (layer F.Cu) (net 3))
 (segment (start 89.37 27.97) (end 89.33 30.07) (width 1) (layer F.Cu) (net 4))
 (segment (start 86.73 30.75) (end 89.33 30.07) (width 1) (layer F.Cu) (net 4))
 (segment (start 86.53 28.715) (end 86.73 30.75) (width 1) (layer F.Cu) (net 4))
 (segment (start 75.25 28.71) (end 73.355753 30.194247) (width 1) (layer F.Cu) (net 4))
 (segment (start 86.53 28.715) (end 75.25 28.71) (width 1) (layer F.Cu) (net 4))
 (segment (start 89.25 41.97) (end 89.34 44.19) (width 1) (layer F.Cu) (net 4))
 (segment (start 86.97 44.9) (end 89.34 44.19) (width 1) (layer F.Cu) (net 4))
 (segment (start 86.97 44.9) (end 86.53 42.845) (width 1) (layer F.Cu) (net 4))
 (segment (start 86.53 42.845) (end 73.359503 42.757583) (width 1) (layer F.Cu) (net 4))
 (segment (start 73.355753 30.194247) (end 73.359503 42.757583) (width 1) (layer F.Cu) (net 4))
 (segment (start 73.359503 42.757583) (end 73.4 48.04) (width 1) (layer F.Cu) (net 4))
 (segment (start 73.4 48.04) (end 74.98712 51.07356) (width 1) (layer F.Cu) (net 4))
 (segment (start 78.17 32.74) (end 86.73 34.05) (width 1) (layer F.Cu) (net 5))
 (segment (start 86.73 34.05) (end 89.33 33.77) (width 1) (layer F.Cu) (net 5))
 (segment (start 78.18 46.63) (end 86.97 48.2) (width 1) (layer F.Cu) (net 8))
 (segment (start 86.97 48.2) (end 89.34 47.89) (width 1) (layer F.Cu) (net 8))
 (segment (start 92.27 27.97) (end 92.33 30.07) (width 1) (layer F.Cu) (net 6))
 (segment (start 91.6 22.56) (end 92.25 25.01) (width 1) (layer F.Cu) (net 6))
 (segment (start 92.25 25.01) (end 92.27 27.97) (width 1) (layer F.Cu) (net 6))
 (segment (start 78.17 22.84) (end 89.06 22.56) (width 1) (layer F.Cu) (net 7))
 (segment (start 92.15 41.97) (end 92.34 44.19) (width 1) (layer F.Cu) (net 9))
 (segment (start 92.2 39.06) (end 92.15 41.97) (width 1) (layer F.Cu) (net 9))
 (segment (start 91.56 36.67) (end 92.2 39.06) (width 1) (layer F.Cu) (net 9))
 (segment (start 78.18 36.73) (end 89.02 36.67) (width 1) (layer F.Cu) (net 10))
 (segment (start 90.52 51.04) (end 92.35 49.39) (width 0.25) (layer F.Cu) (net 1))
 (segment (start 92.35 49.39) (end 92.34 47.89) (width 0.25) (layer F.Cu) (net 1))
 (segment (start 87.68712 51.07356) (end 90.52 51.04) (width 0.25) (layer F.Cu) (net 1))
 (segment (start 93.19 35.05) (end 93.21 49.85) (width 0.25) (layer F.Cu) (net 2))
 (segment (start 93.21 49.85) (end 90.27 52.83) (width 0.25) (layer F.Cu) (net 2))
 (segment (start 90.27 52.83) (end 86.32 52.81) (width 0.25) (layer F.Cu) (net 2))
 (segment (start 86.32 52.81) (end 85.14712 51.07356) (width 0.25) (layer F.Cu) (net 2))
 (segment (start 93.19 35.05) (end 92.33 33.77) (width 0.25) (layer F.Cu) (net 2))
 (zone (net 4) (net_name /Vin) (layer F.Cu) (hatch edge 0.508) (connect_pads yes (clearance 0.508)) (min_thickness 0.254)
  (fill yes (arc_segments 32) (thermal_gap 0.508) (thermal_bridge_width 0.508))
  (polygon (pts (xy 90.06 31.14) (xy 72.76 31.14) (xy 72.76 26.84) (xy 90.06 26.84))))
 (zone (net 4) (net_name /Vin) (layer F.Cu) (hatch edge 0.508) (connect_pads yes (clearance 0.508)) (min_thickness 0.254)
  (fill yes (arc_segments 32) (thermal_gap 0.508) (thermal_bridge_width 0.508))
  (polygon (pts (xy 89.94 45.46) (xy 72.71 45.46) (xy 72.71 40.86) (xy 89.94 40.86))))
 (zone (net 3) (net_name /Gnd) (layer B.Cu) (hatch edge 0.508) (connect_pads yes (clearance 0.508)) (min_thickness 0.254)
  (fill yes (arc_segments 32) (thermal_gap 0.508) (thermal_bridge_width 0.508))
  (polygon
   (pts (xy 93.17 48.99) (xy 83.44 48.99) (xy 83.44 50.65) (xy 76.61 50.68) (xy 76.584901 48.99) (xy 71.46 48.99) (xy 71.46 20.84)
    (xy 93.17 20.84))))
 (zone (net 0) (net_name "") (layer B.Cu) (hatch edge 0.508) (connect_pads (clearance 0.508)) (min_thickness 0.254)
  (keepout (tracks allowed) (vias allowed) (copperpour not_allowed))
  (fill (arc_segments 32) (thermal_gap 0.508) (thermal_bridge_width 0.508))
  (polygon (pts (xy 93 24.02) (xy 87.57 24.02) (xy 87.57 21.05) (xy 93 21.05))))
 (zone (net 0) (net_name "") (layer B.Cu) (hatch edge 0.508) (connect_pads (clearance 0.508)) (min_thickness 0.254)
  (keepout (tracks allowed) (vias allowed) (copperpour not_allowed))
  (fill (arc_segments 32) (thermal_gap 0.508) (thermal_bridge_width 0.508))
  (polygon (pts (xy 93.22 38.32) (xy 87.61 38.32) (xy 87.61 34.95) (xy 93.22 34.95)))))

